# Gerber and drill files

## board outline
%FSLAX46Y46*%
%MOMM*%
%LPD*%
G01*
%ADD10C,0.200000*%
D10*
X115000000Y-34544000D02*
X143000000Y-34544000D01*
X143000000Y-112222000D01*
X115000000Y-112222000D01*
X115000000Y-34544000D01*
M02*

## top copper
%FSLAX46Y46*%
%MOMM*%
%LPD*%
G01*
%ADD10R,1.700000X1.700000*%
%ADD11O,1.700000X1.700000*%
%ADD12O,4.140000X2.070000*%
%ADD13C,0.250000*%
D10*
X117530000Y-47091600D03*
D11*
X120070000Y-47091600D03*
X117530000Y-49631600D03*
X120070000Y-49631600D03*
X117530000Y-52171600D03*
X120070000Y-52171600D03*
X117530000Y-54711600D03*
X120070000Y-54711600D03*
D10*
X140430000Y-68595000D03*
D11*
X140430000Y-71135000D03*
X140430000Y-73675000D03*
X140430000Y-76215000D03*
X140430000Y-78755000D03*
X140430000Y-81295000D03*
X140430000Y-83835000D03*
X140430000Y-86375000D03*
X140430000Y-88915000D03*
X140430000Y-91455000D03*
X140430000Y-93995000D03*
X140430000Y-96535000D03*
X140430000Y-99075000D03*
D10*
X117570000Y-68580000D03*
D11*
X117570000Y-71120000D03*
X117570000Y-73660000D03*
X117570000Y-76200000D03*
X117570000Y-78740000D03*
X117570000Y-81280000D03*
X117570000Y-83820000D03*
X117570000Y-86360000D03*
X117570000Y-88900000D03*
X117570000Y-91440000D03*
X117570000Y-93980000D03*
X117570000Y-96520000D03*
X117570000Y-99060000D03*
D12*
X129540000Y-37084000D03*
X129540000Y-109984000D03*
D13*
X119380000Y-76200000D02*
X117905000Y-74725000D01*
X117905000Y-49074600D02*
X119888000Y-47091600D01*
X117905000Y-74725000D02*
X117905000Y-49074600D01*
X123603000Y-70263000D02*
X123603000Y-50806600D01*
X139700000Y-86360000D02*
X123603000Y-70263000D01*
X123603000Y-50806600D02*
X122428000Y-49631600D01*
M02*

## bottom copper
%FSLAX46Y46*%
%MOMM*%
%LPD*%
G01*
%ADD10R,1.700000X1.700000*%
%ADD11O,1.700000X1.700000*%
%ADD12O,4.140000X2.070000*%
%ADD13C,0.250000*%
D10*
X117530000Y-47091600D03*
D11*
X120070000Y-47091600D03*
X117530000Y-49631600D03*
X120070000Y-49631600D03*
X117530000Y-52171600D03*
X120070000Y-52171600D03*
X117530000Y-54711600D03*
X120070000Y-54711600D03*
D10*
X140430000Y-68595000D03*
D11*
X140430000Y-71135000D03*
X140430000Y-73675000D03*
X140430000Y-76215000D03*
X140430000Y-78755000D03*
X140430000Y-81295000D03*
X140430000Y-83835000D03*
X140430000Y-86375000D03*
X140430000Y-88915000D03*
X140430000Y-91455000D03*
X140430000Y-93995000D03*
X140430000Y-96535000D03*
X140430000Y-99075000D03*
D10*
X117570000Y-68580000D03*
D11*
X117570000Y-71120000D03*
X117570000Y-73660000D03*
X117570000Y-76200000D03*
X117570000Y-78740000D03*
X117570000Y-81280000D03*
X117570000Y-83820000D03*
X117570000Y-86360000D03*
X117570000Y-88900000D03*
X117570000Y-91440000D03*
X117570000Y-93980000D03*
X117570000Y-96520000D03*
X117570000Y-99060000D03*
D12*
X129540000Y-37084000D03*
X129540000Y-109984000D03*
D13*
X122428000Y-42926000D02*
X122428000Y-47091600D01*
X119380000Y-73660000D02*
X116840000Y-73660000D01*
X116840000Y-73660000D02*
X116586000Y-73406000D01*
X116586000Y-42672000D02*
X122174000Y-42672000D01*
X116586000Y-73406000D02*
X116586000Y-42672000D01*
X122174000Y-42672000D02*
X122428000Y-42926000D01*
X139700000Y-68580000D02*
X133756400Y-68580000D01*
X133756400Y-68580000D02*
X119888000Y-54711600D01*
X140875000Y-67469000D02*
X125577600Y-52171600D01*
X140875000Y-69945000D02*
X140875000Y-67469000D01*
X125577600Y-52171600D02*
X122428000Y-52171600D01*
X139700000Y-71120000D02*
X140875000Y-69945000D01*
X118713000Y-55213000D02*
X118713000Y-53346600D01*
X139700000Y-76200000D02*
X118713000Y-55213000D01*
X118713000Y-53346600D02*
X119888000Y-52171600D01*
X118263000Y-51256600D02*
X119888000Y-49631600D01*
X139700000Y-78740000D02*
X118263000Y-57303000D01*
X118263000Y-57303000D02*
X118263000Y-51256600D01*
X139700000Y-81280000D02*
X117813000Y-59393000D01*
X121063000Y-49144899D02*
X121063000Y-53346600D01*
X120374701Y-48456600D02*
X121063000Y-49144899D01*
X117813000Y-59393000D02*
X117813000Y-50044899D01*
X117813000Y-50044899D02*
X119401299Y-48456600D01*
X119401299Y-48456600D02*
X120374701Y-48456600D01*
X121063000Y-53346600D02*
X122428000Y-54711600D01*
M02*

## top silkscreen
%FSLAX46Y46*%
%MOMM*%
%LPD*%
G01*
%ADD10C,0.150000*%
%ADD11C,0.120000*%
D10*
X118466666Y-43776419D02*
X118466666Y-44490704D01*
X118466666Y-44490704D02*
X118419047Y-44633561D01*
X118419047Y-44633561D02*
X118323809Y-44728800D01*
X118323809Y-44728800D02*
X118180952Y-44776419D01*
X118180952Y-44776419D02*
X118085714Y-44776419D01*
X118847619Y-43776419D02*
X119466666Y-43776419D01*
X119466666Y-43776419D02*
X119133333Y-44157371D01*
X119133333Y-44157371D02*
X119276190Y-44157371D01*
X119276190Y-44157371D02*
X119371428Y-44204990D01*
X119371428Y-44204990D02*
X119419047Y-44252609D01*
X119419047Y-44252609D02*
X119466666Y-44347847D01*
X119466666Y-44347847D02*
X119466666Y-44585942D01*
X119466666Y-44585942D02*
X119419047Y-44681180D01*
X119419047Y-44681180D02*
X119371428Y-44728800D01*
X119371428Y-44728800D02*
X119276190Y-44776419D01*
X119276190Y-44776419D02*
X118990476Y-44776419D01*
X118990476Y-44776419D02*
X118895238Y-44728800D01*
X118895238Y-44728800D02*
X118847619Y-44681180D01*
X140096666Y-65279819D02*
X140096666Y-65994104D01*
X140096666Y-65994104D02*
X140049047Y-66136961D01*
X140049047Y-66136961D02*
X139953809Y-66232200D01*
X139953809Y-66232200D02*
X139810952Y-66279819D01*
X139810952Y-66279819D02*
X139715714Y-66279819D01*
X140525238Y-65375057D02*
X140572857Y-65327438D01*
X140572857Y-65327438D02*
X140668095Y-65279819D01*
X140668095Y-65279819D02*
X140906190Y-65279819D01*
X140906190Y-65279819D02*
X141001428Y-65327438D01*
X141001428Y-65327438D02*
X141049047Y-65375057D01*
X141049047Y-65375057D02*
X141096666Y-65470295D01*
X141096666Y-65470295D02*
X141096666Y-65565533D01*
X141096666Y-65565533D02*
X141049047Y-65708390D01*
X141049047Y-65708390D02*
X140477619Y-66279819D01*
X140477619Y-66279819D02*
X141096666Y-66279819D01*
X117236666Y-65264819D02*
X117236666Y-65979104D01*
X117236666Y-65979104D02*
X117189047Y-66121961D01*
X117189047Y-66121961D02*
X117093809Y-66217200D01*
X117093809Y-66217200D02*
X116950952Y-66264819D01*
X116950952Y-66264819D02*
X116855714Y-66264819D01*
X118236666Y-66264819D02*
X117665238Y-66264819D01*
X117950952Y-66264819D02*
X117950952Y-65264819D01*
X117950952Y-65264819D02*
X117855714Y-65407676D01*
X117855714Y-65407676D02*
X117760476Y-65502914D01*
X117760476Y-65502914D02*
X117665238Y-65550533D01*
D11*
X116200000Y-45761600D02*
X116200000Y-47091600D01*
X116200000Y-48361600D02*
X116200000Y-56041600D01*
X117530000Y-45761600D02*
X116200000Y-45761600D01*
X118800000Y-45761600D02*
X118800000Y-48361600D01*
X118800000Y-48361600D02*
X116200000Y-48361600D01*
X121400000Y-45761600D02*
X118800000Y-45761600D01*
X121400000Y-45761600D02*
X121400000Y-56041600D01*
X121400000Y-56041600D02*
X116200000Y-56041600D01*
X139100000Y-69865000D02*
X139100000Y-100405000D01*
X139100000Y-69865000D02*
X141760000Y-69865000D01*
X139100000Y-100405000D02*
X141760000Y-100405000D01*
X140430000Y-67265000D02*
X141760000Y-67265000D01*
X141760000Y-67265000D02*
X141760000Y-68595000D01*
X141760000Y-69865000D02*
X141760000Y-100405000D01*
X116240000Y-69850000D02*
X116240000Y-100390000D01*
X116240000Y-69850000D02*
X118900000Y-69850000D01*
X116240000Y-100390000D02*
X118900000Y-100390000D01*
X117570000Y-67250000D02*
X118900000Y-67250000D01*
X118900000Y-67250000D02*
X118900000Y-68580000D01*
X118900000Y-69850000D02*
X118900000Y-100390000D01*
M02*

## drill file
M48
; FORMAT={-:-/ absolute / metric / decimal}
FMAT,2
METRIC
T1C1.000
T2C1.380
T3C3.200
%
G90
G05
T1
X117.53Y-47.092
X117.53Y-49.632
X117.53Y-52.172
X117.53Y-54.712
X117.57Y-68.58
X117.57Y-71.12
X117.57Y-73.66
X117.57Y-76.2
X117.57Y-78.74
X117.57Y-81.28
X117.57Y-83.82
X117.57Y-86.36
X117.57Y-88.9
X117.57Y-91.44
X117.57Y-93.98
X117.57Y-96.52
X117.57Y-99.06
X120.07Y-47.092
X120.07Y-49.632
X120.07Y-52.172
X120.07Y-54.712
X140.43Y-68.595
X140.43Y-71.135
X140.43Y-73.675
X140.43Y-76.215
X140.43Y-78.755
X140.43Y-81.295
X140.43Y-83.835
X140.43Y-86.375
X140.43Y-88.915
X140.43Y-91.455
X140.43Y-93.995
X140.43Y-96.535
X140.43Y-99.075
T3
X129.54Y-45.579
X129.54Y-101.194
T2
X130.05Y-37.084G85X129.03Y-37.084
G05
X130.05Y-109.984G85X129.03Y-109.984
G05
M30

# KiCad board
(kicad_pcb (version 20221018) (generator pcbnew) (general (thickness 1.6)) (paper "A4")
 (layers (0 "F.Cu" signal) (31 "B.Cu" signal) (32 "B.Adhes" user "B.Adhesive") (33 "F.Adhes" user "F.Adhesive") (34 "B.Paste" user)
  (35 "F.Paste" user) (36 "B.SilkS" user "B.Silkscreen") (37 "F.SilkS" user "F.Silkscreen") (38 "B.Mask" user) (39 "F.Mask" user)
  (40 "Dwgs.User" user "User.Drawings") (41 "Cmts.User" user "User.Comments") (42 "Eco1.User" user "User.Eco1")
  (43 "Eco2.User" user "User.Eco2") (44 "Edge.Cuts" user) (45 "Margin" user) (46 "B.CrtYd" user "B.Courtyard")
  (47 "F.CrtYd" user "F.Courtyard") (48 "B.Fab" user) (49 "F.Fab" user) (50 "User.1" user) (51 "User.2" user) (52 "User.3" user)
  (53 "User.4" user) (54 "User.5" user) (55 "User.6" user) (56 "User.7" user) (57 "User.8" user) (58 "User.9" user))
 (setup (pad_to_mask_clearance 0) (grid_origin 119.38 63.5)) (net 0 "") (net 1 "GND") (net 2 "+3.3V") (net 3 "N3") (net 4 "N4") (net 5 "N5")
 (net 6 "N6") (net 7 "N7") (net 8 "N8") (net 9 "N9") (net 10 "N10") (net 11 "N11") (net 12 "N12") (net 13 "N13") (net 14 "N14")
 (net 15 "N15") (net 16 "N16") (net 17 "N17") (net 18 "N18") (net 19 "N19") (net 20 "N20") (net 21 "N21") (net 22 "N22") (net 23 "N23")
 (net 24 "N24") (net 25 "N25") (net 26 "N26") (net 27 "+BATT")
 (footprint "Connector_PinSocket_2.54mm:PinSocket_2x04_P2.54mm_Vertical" (layer "F.Cu") (at 120.11 47.0916)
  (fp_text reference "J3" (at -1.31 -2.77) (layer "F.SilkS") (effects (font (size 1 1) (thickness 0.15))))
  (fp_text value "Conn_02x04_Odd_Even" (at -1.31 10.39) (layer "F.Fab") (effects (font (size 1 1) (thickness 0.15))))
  (fp_line (start -3.91 -1.33) (end -3.91 0) (stroke (width 0.12) (type solid)) (layer "F.SilkS"))
  (fp_line (start -3.91 1.27) (end -3.91 8.95) (stroke (width 0.12) (type solid)) (layer "F.SilkS"))
  (fp_line (start -2.58 -1.33) (end -3.91 -1.33) (stroke (width 0.12) (type solid)) (layer "F.SilkS"))
  (fp_line (start -1.31 -1.33) (end -1.31 1.27) (stroke (width 0.12) (type solid)) (layer "F.SilkS"))
  (fp_line (start -1.31 1.27) (end -3.91 1.27) (stroke (width 0.12) (type solid)) (layer "F.SilkS"))
  (fp_line (start 1.29 -1.33) (end -1.31 -1.33) (stroke (width 0.12) (type solid)) (layer "F.SilkS"))
  (fp_line (start 1.29 -1.33) (end 1.29 8.95) (stroke (width 0.12) (type solid)) (layer "F.SilkS"))
  (fp_line (start 1.29 8.95) (end -3.91 8.95) (stroke (width 0.12) (type solid)) (layer "F.SilkS"))
  (pad "1" thru_hole rect (at -2.58 0) (size 1.7 1.7) (drill 1) (layers "*.Cu" "*.Mask") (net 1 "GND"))
  (pad "2" thru_hole oval (at -0.04 0) (size 1.7 1.7) (drill 1) (layers "*.Cu" "*.Mask") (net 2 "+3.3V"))
  (pad "3" thru_hole oval (at -2.58 2.54) (size 1.7 1.7) (drill 1) (layers "*.Cu" "*.Mask") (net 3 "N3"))
  (pad "4" thru_hole oval (at -0.04 2.54) (size 1.7 1.7) (drill 1) (layers "*.Cu" "*.Mask") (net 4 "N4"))
  (pad "5" thru_hole oval (at -2.58 5.08) (size 1.7 1.7) (drill 1) (layers "*.Cu" "*.Mask") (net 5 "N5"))
  (pad "6" thru_hole oval (at -0.04 5.08) (size 1.7 1.7) (drill 1) (layers "*.Cu" "*.Mask") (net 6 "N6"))
  (pad "7" thru_hole oval (at -2.58 7.62) (size 1.7 1.7) (drill 1) (layers "*.Cu" "*.Mask") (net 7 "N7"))
  (pad "8" thru_hole oval (at -0.04 7.62) (size 1.7 1.7) (drill 1) (layers "*.Cu" "*.Mask") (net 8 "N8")))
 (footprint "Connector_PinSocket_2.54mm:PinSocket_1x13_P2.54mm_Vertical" (layer "F.Cu") (at 140.43 68.595)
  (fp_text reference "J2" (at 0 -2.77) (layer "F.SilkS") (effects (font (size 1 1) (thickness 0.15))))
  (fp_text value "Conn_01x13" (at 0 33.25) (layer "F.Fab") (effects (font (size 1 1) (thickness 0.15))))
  (fp_line (start -1.33 1.27) (end -1.33 31.81) (stroke (width 0.12) (type solid)) (layer "F.SilkS"))
  (fp_line (start -1.33 1.27) (end 1.33 1.27) (stroke (width 0.12) (type solid)) (layer "F.SilkS"))
  (fp_line (start -1.33 31.81) (end 1.33 31.81) (stroke (width 0.12) (type solid)) (layer "F.SilkS"))
  (fp_line (start 0 -1.33) (end 1.33 -1.33) (stroke (width 0.12) (type solid)) (layer "F.SilkS"))
  (fp_line (start 1.33 -1.33) (end 1.33 0) (stroke (width 0.12) (type solid)) (layer "F.SilkS"))
  (fp_line (start 1.33 1.27) (end 1.33 31.81) (stroke (width 0.12) (type solid)) (layer "F.SilkS"))
  (pad "1" thru_hole rect (at 0 0) (size 1.7 1.7) (drill 1) (layers "*.Cu" "*.Mask") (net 7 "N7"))
  (pad "2" thru_hole oval (at 0 2.54) (size 1.7 1.7) (drill 1) (layers "*.Cu" "*.Mask") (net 6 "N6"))
  (pad "3" thru_hole oval (at 0 5.08) (size 1.7 1.7) (drill 1) (layers "*.Cu" "*.Mask") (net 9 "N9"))
  (pad "4" thru_hole oval (at 0 7.62) (size 1.7 1.7) (drill 1) (layers "*.Cu" "*.Mask") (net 5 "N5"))
  (pad "5" thru_hole oval (at 0 10.16) (size 1.7 1.7) (drill 1) (layers "*.Cu" "*.Mask") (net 3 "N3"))
  (pad "6" thru_hole oval (at 0 12.7) (size 1.7 1.7) (drill 1) (layers "*.Cu" "*.Mask") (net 8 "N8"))
  (pad "7" thru_hole oval (at 0 15.24) (size 1.7 1.7) (drill 1) (layers "*.Cu" "*.Mask") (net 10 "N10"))
  (pad "8" thru_hole oval (at 0 17.78) (size 1.7 1.7) (drill 1) (layers "*.Cu" "*.Mask") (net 4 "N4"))
  (pad "9" thru_hole oval (at 0 20.32) (size 1.7 1.7) (drill 1) (layers "*.Cu" "*.Mask") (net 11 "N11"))
  (pad "10" thru_hole oval (at 0 22.86) (size 1.7 1.7) (drill 1) (layers "*.Cu" "*.Mask") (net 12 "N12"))
  (pad "11" thru_hole oval (at 0 25.4) (size 1.7 1.7) (drill 1) (layers "*.Cu" "*.Mask") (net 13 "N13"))
  (pad "12" thru_hole oval (at 0 27.94) (size 1.7 1.7) (drill 1) (layers "*.Cu" "*.Mask") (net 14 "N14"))
  (pad "13" thru_hole oval (at 0 30.48) (size 1.7 1.7) (drill 1) (layers "*.Cu" "*.Mask") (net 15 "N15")))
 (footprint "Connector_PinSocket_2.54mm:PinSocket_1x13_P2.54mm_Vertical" (layer "F.Cu") (at 117.57 68.58)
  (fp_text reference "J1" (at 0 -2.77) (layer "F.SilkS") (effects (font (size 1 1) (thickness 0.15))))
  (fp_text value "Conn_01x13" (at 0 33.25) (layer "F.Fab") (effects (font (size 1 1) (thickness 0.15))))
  (fp_line (start -1.33 1.27) (end -1.33 31.81) (stroke (width 0.12) (type solid)) (layer "F.SilkS"))
  (fp_line (start -1.33 1.27) (end 1.33 1.27) (stroke (width 0.12) (type solid)) (layer "F.SilkS"))
  (fp_line (start -1.33 31.81) (end 1.33 31.81) (stroke (width 0.12) (type solid)) (layer "F.SilkS"))
  (fp_line (start 0 -1.33) (end 1.33 -1.33) (stroke (width 0.12) (type solid)) (layer "F.SilkS"))
  (fp_line (start 1.33 -1.33) (end 1.33 0) (stroke (width 0.12) (type solid)) (layer "F.SilkS"))
  (fp_line (start 1.33 1.27) (end 1.33 31.81) (stroke (width 0.12) (type solid)) (layer "F.SilkS"))
  (pad "1" thru_hole rect (at 0 0) (size 1.7 1.7) (drill 1) (layers "*.Cu" "*.Mask") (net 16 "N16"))
  (pad "2" thru_hole oval (at 0 2.54) (size 1.7 1.7) (drill 1) (layers "*.Cu" "*.Mask") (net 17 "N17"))
  (pad "3" thru_hole oval (at 0 5.08) (size 1.7 1.7) (drill 1) (layers "*.Cu" "*.Mask") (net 2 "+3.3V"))
  (pad "4" thru_hole oval (at 0 7.62) (size 1.7 1.7) (drill 1) (layers "*.Cu" "*.Mask") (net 1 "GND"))
  (pad "5" thru_hole oval (at 0 10.16) (size 1.7 1.7) (drill 1) (layers "*.Cu" "*.Mask") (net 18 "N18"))
  (pad "6" thru_hole oval (at 0 12.7) (size 1.7 1.7) (drill 1) (layers "*.Cu" "*.Mask") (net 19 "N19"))
  (pad "7" thru_hole oval (at 0 15.24) (size 1.7 1.7) (drill 1) (layers "*.Cu" "*.Mask") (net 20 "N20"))
  (pad "8" thru_hole oval (at 0 17.78) (size 1.7 1.7) (drill 1) (layers "*.Cu" "*.Mask") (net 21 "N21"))
  (pad "9" thru_hole oval (at 0 20.32) (size 1.7 1.7) (drill 1) (layers "*.Cu" "*.Mask") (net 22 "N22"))
  (pad "10" thru_hole oval (at 0 22.86) (size 1.7 1.7) (drill 1) (layers "*.Cu" "*.Mask") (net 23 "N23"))
  (pad "11" thru_hole oval (at 0 25.4) (size 1.7 1.7) (drill 1) (layers "*.Cu" "*.Mask") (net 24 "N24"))
  (pad "12" thru_hole oval (at 0 27.94) (size 1.7 1.7) (drill 1) (layers "*.Cu" "*.Mask") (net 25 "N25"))
  (pad "13" thru_hole oval (at 0 30.48) (size 1.7 1.7) (drill 1) (layers "*.Cu" "*.Mask") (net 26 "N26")))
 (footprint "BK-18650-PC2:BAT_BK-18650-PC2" (layer "B.Cu") (at 129.54 73.384 -90)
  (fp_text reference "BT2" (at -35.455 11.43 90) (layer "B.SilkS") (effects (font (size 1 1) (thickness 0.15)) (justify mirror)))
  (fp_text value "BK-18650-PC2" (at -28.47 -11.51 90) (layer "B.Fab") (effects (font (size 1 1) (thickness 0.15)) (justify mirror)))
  (pad "" np_thru_hole circle (at -27.805 0 270) (size 3.2 3.2) (drill 3.2) (layers "*.Cu" "*.Mask"))
  (pad "" np_thru_hole circle (at 27.81 0 270) (size 3.2 3.2) (drill 3.2) (layers "*.Cu" "*.Mask"))
  (pad "+" thru_hole oval (at -36.3 0 270) (size 2.07 4.14) (drill oval 1.38 2.4) (layers "*.Cu" "*.Mask") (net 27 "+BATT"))
  (pad "-" thru_hole oval (at 36.6 0 270) (size 2.07 4.14) (drill oval 1.38 2.4) (layers "*.Cu" "*.Mask") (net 1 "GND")))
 (gr_rect (start 115 34.544) (end 143 112.222) (stroke (width 0.2) (type default)) (fill none) (layer "Edge.Cuts"))
 (segment (start 122.428 42.926) (end 122.428 47.0916) (width 0.25) (layer "B.Cu") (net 2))
 (segment (start 119.38 73.66) (end 116.84 73.66) (width 0.25) (layer "B.Cu") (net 2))
 (segment (start 116.84 73.66) (end 116.586 73.406) (width 0.25) (layer "B.Cu") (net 2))
 (segment (start 116.586 42.672) (end 122.174 42.672) (width 0.25) (layer "B.Cu") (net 2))
 (segment (start 116.586 73.406) (end 116.586 42.672) (width 0.25) (layer "B.Cu") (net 2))
 (segment (start 122.174 42.672) (end 122.428 42.926) (width 0.25) (layer "B.Cu") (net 2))
 (segment (start 119.38 76.2) (end 117.905 74.725) (width 0.25) (layer "F.Cu") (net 1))
 (segment (start 117.905 49.0746) (end 119.888 47.0916) (width 0.25) (layer "F.Cu") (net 1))
 (segment (start 117.905 74.725) (end 117.905 49.0746) (width 0.25) (layer "F.Cu") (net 1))
 (segment (start 139.7 68.58) (end 133.7564 68.58) (width 0.25) (layer "B.Cu") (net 7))
 (segment (start 133.7564 68.58) (end 119.888 54.7116) (width 0.25) (layer "B.Cu") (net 7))
 (segment (start 140.875 67.469) (end 125.5776 52.1716) (width 0.25) (layer "B.Cu") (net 6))
 (segment (start 140.875 69.945) (end 140.875 67.469) (width 0.25) (layer "B.Cu") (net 6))
 (segment (start 125.5776 52.1716) (end 122.428 52.1716) (width 0.25) (layer "B.Cu") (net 6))
 (segment (start 139.7 71.12) (end 140.875 69.945) (width 0.25) (layer "B.Cu") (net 6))
 (segment (start 118.713 55.213) (end 118.713 53.3466) (width 0.25) (layer "B.Cu") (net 5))
 (segment (start 139.7 76.2) (end 118.713 55.213) (width 0.25) (layer "B.Cu") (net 5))
 (segment (start 118.713 53.3466) (end 119.888 52.1716) (width 0.25) (layer "B.Cu") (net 5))
 (segment (start 118.263 51.2566) (end 119.888 49.6316) (width 0.25) (layer "B.Cu") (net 3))
 (segment (start 139.7 78.74) (end 118.263 57.303) (width 0.25) (layer "B.Cu") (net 3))
 (segment (start 118.263 57.303) (end 118.263 51.2566) (width 0.25) (layer "B.Cu") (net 3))
 (segment (start 139.7 81.28) (end 117.813 59.393) (width 0.25) (layer "B.Cu") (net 8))
 (segment (start 121.063 49.144899) (end 121.063 53.3466) (width 0.25) (layer "B.Cu") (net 8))
 (segment (start 120.374701 48.4566) (end 121.063 49.144899) (width 0.25) (layer "B.Cu") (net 8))
 (segment (start 117.813 59.393) (end 117.813 50.044899) (width 0.25) (layer "B.Cu") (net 8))
 (segment (start 117.813 50.044899) (end 119.401299 48.4566) (width 0.25) (layer "B.Cu") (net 8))
 (segment (start 119.401299 48.4566) (end 120.374701 48.4566) (width 0.25) (layer "B.Cu") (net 8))
 (segment (start 121.063 53.3466) (end 122.428 54.7116) (width 0.25) (layer "B.Cu") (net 8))
 (segment (start 123.603 70.263) (end 123.603 50.8066) (width 0.25) (layer "F.Cu") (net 4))
 (segment (start 139.7 86.36) (end 123.603 70.263) (width 0.25) (layer "F.Cu") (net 4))
 (segment (start 123.603 50.8066) (end 122.428 49.6316) (width 0.25) (layer "F.Cu") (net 4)))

